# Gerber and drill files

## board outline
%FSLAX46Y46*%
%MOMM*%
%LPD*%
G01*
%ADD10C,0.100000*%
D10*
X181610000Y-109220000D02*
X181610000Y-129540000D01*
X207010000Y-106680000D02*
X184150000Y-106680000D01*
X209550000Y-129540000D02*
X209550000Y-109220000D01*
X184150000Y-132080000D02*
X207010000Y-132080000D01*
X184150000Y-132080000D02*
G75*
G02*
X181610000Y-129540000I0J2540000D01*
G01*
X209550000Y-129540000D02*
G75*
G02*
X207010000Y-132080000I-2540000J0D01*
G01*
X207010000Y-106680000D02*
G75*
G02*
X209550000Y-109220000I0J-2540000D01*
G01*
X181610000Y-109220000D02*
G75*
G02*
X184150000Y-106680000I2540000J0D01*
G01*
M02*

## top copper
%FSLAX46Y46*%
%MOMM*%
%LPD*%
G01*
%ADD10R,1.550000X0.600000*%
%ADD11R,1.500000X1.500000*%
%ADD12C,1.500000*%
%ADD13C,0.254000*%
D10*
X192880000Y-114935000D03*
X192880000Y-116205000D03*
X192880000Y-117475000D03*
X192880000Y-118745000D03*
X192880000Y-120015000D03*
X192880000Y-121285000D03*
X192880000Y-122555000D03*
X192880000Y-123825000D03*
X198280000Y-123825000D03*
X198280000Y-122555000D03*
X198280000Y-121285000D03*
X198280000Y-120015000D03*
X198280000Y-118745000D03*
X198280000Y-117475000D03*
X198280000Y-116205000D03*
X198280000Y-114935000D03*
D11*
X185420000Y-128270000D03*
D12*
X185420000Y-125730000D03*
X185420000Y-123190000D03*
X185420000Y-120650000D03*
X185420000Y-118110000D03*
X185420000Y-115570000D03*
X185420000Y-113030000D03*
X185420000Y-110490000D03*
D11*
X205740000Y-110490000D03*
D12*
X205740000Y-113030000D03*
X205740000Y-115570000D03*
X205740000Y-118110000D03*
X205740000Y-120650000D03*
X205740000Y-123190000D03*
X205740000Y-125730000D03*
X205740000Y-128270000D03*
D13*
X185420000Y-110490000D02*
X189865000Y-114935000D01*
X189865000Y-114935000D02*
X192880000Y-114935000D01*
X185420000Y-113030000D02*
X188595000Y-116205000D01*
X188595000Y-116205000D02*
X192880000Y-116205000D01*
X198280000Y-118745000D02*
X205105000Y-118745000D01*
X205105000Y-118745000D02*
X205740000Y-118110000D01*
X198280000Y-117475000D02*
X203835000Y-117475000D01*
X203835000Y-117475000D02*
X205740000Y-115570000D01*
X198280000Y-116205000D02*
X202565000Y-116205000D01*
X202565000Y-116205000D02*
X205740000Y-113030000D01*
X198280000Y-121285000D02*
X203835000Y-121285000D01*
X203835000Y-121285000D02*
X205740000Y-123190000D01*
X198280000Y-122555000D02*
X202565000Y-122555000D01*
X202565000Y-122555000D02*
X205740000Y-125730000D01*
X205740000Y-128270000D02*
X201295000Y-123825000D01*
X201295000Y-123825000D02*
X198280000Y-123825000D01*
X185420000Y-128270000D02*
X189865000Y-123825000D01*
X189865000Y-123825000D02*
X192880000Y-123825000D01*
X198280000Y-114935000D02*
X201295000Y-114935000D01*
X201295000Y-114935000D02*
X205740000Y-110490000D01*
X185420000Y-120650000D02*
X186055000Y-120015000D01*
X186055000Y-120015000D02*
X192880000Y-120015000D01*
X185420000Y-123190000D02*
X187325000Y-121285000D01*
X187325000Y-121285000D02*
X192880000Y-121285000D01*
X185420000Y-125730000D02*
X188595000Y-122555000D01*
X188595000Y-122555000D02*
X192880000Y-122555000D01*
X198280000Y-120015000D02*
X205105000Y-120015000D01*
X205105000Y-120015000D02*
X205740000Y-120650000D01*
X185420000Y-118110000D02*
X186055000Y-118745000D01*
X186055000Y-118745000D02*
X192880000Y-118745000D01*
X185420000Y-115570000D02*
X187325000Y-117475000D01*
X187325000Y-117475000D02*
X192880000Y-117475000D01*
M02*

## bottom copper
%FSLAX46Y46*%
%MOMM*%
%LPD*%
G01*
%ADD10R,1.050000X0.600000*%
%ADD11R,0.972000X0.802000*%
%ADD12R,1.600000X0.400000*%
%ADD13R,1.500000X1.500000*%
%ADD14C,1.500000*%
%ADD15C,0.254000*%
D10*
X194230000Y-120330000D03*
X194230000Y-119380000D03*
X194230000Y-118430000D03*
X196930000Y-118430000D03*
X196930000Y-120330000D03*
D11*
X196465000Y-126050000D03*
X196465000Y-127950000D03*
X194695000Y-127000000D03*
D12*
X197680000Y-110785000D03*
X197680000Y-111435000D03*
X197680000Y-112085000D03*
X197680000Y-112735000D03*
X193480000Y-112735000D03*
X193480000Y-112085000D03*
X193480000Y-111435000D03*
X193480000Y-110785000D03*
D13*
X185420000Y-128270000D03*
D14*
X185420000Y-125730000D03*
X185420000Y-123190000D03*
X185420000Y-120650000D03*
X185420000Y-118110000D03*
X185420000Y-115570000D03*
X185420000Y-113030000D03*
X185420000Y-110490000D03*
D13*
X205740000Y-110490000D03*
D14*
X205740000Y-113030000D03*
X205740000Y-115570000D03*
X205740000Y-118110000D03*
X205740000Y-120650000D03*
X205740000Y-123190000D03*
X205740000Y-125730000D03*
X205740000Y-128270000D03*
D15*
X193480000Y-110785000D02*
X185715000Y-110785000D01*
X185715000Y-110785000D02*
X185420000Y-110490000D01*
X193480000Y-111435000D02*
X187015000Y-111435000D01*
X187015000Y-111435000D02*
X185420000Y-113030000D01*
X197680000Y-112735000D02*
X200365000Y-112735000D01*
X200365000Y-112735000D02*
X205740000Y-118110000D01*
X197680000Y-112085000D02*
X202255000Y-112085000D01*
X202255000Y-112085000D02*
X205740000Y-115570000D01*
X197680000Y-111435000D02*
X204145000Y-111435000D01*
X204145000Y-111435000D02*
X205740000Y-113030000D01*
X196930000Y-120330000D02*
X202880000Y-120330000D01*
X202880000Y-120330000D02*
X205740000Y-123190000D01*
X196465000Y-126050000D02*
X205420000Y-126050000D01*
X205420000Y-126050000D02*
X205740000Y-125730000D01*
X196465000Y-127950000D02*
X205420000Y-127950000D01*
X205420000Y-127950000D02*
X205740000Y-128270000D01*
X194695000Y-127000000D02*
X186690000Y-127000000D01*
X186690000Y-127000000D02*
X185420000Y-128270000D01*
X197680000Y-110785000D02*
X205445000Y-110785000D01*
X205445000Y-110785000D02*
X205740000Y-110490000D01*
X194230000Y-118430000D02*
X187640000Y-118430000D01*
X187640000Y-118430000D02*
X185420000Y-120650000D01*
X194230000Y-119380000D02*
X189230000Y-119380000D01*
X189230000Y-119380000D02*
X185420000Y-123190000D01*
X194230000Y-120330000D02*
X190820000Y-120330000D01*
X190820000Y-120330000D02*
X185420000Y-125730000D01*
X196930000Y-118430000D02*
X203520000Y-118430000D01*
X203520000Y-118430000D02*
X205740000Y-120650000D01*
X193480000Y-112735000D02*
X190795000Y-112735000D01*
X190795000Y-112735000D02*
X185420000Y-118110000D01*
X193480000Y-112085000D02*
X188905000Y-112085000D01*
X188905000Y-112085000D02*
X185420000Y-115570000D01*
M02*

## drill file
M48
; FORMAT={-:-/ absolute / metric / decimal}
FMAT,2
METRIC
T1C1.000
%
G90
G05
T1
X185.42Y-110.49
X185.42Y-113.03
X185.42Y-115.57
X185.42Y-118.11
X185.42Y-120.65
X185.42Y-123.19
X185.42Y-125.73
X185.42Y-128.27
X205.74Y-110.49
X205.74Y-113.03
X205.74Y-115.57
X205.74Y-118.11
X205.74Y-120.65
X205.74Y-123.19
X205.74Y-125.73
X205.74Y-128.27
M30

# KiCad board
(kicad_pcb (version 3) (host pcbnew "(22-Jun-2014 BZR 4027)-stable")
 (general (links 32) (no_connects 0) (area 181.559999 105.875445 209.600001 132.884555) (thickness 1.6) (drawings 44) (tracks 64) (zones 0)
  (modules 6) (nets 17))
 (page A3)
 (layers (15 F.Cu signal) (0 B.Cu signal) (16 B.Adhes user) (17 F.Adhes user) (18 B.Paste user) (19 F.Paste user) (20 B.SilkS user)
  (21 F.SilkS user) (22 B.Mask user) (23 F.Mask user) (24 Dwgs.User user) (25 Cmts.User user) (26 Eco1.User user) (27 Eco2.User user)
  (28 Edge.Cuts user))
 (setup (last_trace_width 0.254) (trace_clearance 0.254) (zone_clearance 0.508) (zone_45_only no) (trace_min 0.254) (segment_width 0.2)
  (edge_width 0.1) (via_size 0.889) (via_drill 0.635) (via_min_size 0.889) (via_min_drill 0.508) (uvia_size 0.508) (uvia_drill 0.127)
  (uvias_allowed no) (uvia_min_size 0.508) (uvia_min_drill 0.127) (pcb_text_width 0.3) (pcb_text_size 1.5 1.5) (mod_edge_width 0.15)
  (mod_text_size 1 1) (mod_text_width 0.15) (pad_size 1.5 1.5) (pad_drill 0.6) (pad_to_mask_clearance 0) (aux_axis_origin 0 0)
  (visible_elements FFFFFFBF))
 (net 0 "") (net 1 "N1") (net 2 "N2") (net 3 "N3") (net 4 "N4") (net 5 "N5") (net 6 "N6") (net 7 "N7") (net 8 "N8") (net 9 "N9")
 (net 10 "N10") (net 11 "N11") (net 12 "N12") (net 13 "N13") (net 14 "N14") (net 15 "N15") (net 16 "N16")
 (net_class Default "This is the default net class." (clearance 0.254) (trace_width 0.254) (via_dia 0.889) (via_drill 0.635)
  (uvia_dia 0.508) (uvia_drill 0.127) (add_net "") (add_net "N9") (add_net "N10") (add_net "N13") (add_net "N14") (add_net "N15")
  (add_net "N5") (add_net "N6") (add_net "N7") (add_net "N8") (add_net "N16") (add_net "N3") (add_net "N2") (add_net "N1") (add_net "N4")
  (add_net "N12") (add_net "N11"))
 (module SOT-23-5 (layer B.Cu) (at 195.58 119.38 90) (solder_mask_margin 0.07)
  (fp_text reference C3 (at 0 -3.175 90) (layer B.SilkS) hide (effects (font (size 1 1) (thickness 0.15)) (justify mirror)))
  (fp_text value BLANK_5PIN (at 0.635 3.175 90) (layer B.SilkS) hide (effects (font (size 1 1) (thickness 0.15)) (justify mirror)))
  (pad 1 smd rect (at -0.95 -1.35 90) (size 0.6 1.05) (layers B.Cu B.Paste B.Mask) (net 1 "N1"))
  (pad 2 smd rect (at 0 -1.35 90) (size 0.6 1.05) (layers B.Cu B.Paste B.Mask) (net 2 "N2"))
  (pad 3 smd rect (at 0.95 -1.35 90) (size 0.6 1.05) (layers B.Cu B.Paste B.Mask) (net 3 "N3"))
  (pad 4 smd rect (at 0.95 1.35 90) (size 0.6 1.05) (layers B.Cu B.Paste B.Mask) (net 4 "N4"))
  (pad 5 smd rect (at -0.95 1.35 90) (size 0.6 1.05) (layers B.Cu B.Paste B.Mask) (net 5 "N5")))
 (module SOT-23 (layer B.Cu) (at 195.58 127 270) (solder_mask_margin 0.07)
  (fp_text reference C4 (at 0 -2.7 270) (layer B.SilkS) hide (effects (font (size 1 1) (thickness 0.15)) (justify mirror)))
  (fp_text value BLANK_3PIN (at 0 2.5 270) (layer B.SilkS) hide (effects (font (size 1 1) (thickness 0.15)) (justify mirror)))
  (pad 1 smd rect (at -0.95 -0.885 270) (size 0.802 0.972) (layers B.Cu B.Paste B.Mask) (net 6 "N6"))
  (pad 2 smd rect (at 0.95 -0.885 270) (size 0.802 0.972) (layers B.Cu B.Paste B.Mask) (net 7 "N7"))
  (pad 3 smd rect (at 0 0.885 270) (size 0.802 0.972) (layers B.Cu B.Paste B.Mask) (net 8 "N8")))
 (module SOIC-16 (layer F.Cu) (at 195.58 119.38 270)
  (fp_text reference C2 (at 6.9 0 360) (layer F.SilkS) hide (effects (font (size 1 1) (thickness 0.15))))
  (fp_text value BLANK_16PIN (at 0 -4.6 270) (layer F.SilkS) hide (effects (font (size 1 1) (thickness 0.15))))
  (pad 1 smd rect (at -4.445 2.7 270) (size 0.6 1.55) (layers F.Cu F.Paste F.Mask) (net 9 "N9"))
  (pad 2 smd rect (at -3.175 2.7 270) (size 0.6 1.55) (layers F.Cu F.Paste F.Mask) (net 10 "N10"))
  (pad 3 smd rect (at -1.905 2.7 270) (size 0.6 1.55) (layers F.Cu F.Paste F.Mask) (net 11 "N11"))
  (pad 4 smd rect (at -0.635 2.7 270) (size 0.6 1.55) (layers F.Cu F.Paste F.Mask) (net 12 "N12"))
  (pad 5 smd rect (at 0.635 2.7 270) (size 0.6 1.55) (layers F.Cu F.Paste F.Mask) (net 3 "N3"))
  (pad 6 smd rect (at 1.905 2.7 270) (size 0.6 1.55) (layers F.Cu F.Paste F.Mask) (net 2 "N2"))
  (pad 7 smd rect (at 3.175 2.7 270) (size 0.6 1.55) (layers F.Cu F.Paste F.Mask) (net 1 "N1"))
  (pad 8 smd rect (at 4.445 2.7 270) (size 0.6 1.55) (layers F.Cu F.Paste F.Mask) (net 8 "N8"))
  (pad 9 smd rect (at 4.445 -2.7 270) (size 0.6 1.55) (layers F.Cu F.Paste F.Mask) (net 7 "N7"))
  (pad 10 smd rect (at 3.175 -2.7 270) (size 0.6 1.55) (layers F.Cu F.Paste F.Mask) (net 6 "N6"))
  (pad 11 smd rect (at 1.905 -2.7 270) (size 0.6 1.55) (layers F.Cu F.Paste F.Mask) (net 5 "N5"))
  (pad 12 smd rect (at 0.635 -2.7 270) (size 0.6 1.55) (layers F.Cu F.Paste F.Mask) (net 4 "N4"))
  (pad 13 smd rect (at -0.635 -2.7 270) (size 0.6 1.55) (layers F.Cu F.Paste F.Mask) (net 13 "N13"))
  (pad 14 smd rect (at -1.905 -2.7 270) (size 0.6 1.55) (layers F.Cu F.Paste F.Mask) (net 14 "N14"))
  (pad 15 smd rect (at -3.175 -2.7 270) (size 0.6 1.55) (layers F.Cu F.Paste F.Mask) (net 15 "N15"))
  (pad 16 smd rect (at -4.445 -2.7 270) (size 0.6 1.55) (layers F.Cu F.Paste F.Mask) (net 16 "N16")))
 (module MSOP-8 (layer B.Cu) (at 195.58 111.76 270) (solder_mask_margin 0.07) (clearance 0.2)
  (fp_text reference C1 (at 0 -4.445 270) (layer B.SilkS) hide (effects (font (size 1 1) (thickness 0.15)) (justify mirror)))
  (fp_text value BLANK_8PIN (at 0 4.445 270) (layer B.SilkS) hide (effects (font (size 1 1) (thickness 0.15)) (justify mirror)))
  (pad 1 smd rect (at -0.975 -2.1 270) (size 0.4 1.6) (layers B.Cu B.Paste B.Mask) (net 16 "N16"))
  (pad 2 smd rect (at -0.325 -2.1 270) (size 0.4 1.6) (layers B.Cu B.Paste B.Mask) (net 15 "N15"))
  (pad 3 smd rect (at 0.325 -2.1 270) (size 0.4 1.6) (layers B.Cu B.Paste B.Mask) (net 14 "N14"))
  (pad 4 smd rect (at 0.975 -2.1 270) (size 0.4 1.6) (layers B.Cu B.Paste B.Mask) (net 13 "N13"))
  (pad 5 smd rect (at 0.975 2.1 270) (size 0.4 1.6) (layers B.Cu B.Paste B.Mask) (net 12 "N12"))
  (pad 6 smd rect (at 0.325 2.1 270) (size 0.4 1.6) (layers B.Cu B.Paste B.Mask) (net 11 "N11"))
  (pad 7 smd rect (at -0.325 2.1 270) (size 0.4 1.6) (layers B.Cu B.Paste B.Mask) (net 10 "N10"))
  (pad 8 smd rect (at -0.975 2.1 270) (size 0.4 1.6) (layers B.Cu B.Paste B.Mask) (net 9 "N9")))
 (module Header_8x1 (layer F.Cu) (at 185.42 119.38 90)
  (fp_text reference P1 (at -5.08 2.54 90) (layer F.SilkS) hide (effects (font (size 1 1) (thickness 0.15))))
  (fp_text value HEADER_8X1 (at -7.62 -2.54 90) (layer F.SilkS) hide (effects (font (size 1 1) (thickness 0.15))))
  (pad 1 thru_hole rect (at -8.89 0 90) (size 1.5 1.5) (drill 1) (layers *.Cu *.Mask F.SilkS) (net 8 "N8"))
  (pad 2 thru_hole circle (at -6.35 0 90) (size 1.5 1.5) (drill 1) (layers *.Cu *.Mask F.SilkS) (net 1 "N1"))
  (pad 3 thru_hole circle (at -3.81 0 90) (size 1.5 1.5) (drill 1) (layers *.Cu *.Mask F.SilkS) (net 2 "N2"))
  (pad 4 thru_hole circle (at -1.27 0 90) (size 1.5 1.5) (drill 1) (layers *.Cu *.Mask F.SilkS) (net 3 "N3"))
  (pad 5 thru_hole circle (at 1.27 0 90) (size 1.5 1.5) (drill 1) (layers *.Cu *.Mask F.SilkS) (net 12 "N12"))
  (pad 6 thru_hole circle (at 3.81 0 90) (size 1.5 1.5) (drill 1) (layers *.Cu *.Mask F.SilkS) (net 11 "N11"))
  (pad 7 thru_hole circle (at 6.35 0 90) (size 1.5 1.5) (drill 1) (layers *.Cu *.Mask F.SilkS) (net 10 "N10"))
  (pad 8 thru_hole circle (at 8.89 0 90) (size 1.5 1.5) (drill 1) (layers *.Cu *.Mask F.SilkS) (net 9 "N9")))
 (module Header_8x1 (layer F.Cu) (at 205.74 119.38 270)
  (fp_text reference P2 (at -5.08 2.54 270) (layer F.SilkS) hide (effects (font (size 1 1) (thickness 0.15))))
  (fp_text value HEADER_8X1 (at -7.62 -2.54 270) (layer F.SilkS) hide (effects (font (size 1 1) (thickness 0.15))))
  (pad 1 thru_hole rect (at -8.89 0 270) (size 1.5 1.5) (drill 1) (layers *.Cu *.Mask F.SilkS) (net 16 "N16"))
  (pad 2 thru_hole circle (at -6.35 0 270) (size 1.5 1.5) (drill 1) (layers *.Cu *.Mask F.SilkS) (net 15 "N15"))
  (pad 3 thru_hole circle (at -3.81 0 270) (size 1.5 1.5) (drill 1) (layers *.Cu *.Mask F.SilkS) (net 14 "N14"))
  (pad 4 thru_hole circle (at -1.27 0 270) (size 1.5 1.5) (drill 1) (layers *.Cu *.Mask F.SilkS) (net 13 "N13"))
  (pad 5 thru_hole circle (at 1.27 0 270) (size 1.5 1.5) (drill 1) (layers *.Cu *.Mask F.SilkS) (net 4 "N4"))
  (pad 6 thru_hole circle (at 3.81 0 270) (size 1.5 1.5) (drill 1) (layers *.Cu *.Mask F.SilkS) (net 5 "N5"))
  (pad 7 thru_hole circle (at 6.35 0 270) (size 1.5 1.5) (drill 1) (layers *.Cu *.Mask F.SilkS) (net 6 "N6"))
  (pad 8 thru_hole circle (at 8.89 0 270) (size 1.5 1.5) (drill 1) (layers *.Cu *.Mask F.SilkS) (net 7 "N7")))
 (gr_line (start 181.61 109.22) (end 181.61 129.54) (angle 90) (layer Edge.Cuts) (width 0.1))
 (gr_line (start 207.01 106.68) (end 184.15 106.68) (angle 90) (layer Edge.Cuts) (width 0.1))
 (gr_line (start 209.55 129.54) (end 209.55 109.22) (angle 90) (layer Edge.Cuts) (width 0.1))
 (gr_line (start 184.15 132.08) (end 207.01 132.08) (angle 90) (layer Edge.Cuts) (width 0.1))
 (gr_arc (start 184.15 129.54) (end 184.15 132.08) (angle 90) (layer Edge.Cuts) (width 0.1))
 (gr_arc (start 207.01 129.54) (end 209.55 129.54) (angle 90) (layer Edge.Cuts) (width 0.1))
 (gr_arc (start 207.01 109.22) (end 207.01 106.68) (angle 90) (layer Edge.Cuts) (width 0.1))
 (gr_arc (start 184.15 109.22) (end 181.61 109.22) (angle 90) (layer Edge.Cuts) (width 0.1))
 (segment (start 185.42 110.49) (end 189.865 114.935) (width 0.254) (layer F.Cu) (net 9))
 (segment (start 189.865 114.935) (end 192.88 114.935) (width 0.254) (layer F.Cu) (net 9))
 (segment (start 193.48 110.785) (end 185.715 110.785) (width 0.254) (layer B.Cu) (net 9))
 (segment (start 185.715 110.785) (end 185.42 110.49) (width 0.254) (layer B.Cu) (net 9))
 (segment (start 185.42 113.03) (end 188.595 116.205) (width 0.254) (layer F.Cu) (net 10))
 (segment (start 188.595 116.205) (end 192.88 116.205) (width 0.254) (layer F.Cu) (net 10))
 (segment (start 193.48 111.435) (end 187.015 111.435) (width 0.254) (layer B.Cu) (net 10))
 (segment (start 187.015 111.435) (end 185.42 113.03) (width 0.254) (layer B.Cu) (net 10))
 (segment (start 198.28 118.745) (end 205.105 118.745) (width 0.254) (layer F.Cu) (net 13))
 (segment (start 205.105 118.745) (end 205.74 118.11) (width 0.254) (layer F.Cu) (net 13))
 (segment (start 197.68 112.735) (end 200.365 112.735) (width 0.254) (layer B.Cu) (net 13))
 (segment (start 200.365 112.735) (end 205.74 118.11) (width 0.254) (layer B.Cu) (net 13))
 (segment (start 198.28 117.475) (end 203.835 117.475) (width 0.254) (layer F.Cu) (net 14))
 (segment (start 203.835 117.475) (end 205.74 115.57) (width 0.254) (layer F.Cu) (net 14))
 (segment (start 197.68 112.085) (end 202.255 112.085) (width 0.254) (layer B.Cu) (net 14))
 (segment (start 202.255 112.085) (end 205.74 115.57) (width 0.254) (layer B.Cu) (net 14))
 (segment (start 198.28 116.205) (end 202.565 116.205) (width 0.254) (layer F.Cu) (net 15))
 (segment (start 202.565 116.205) (end 205.74 113.03) (width 0.254) (layer F.Cu) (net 15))
 (segment (start 197.68 111.435) (end 204.145 111.435) (width 0.254) (layer B.Cu) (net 15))
 (segment (start 204.145 111.435) (end 205.74 113.03) (width 0.254) (layer B.Cu) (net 15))
 (segment (start 198.28 121.285) (end 203.835 121.285) (width 0.254) (layer F.Cu) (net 5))
 (segment (start 203.835 121.285) (end 205.74 123.19) (width 0.254) (layer F.Cu) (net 5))
 (segment (start 196.93 120.33) (end 202.88 120.33) (width 0.254) (layer B.Cu) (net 5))
 (segment (start 202.88 120.33) (end 205.74 123.19) (width 0.254) (layer B.Cu) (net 5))
 (segment (start 198.28 122.555) (end 202.565 122.555) (width 0.254) (layer F.Cu) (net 6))
 (segment (start 202.565 122.555) (end 205.74 125.73) (width 0.254) (layer F.Cu) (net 6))
 (segment (start 196.465 126.05) (end 205.42 126.05) (width 0.254) (layer B.Cu) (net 6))
 (segment (start 205.42 126.05) (end 205.74 125.73) (width 0.254) (layer B.Cu) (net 6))
 (segment (start 205.74 128.27) (end 201.295 123.825) (width 0.254) (layer F.Cu) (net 7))
 (segment (start 201.295 123.825) (end 198.28 123.825) (width 0.254) (layer F.Cu) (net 7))
 (segment (start 196.465 127.95) (end 205.42 127.95) (width 0.254) (layer B.Cu) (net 7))
 (segment (start 205.42 127.95) (end 205.74 128.27) (width 0.254) (layer B.Cu) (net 7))
 (segment (start 185.42 128.27) (end 189.865 123.825) (width 0.254) (layer F.Cu) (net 8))
 (segment (start 189.865 123.825) (end 192.88 123.825) (width 0.254) (layer F.Cu) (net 8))
 (segment (start 194.695 127) (end 186.69 127) (width 0.254) (layer B.Cu) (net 8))
 (segment (start 186.69 127) (end 185.42 128.27) (width 0.254) (layer B.Cu) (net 8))
 (segment (start 198.28 114.935) (end 201.295 114.935) (width 0.254) (layer F.Cu) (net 16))
 (segment (start 201.295 114.935) (end 205.74 110.49) (width 0.254) (layer F.Cu) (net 16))
 (segment (start 197.68 110.785) (end 205.445 110.785) (width 0.254) (layer B.Cu) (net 16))
 (segment (start 205.445 110.785) (end 205.74 110.49) (width 0.254) (layer B.Cu) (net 16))
 (segment (start 185.42 120.65) (end 186.055 120.015) (width 0.254) (layer F.Cu) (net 3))
 (segment (start 186.055 120.015) (end 192.88 120.015) (width 0.254) (layer F.Cu) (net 3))
 (segment (start 194.23 118.43) (end 187.64 118.43) (width 0.254) (layer B.Cu) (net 3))
 (segment (start 187.64 118.43) (end 185.42 120.65) (width 0.254) (layer B.Cu) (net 3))
 (segment (start 185.42 123.19) (end 187.325 121.285) (width 0.254) (layer F.Cu) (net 2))
 (segment (start 187.325 121.285) (end 192.88 121.285) (width 0.254) (layer F.Cu) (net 2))
 (segment (start 194.23 119.38) (end 189.23 119.38) (width 0.254) (layer B.Cu) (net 2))
 (segment (start 189.23 119.38) (end 185.42 123.19) (width 0.254) (layer B.Cu) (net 2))
 (segment (start 185.42 125.73) (end 188.595 122.555) (width 0.254) (layer F.Cu) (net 1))
 (segment (start 188.595 122.555) (end 192.88 122.555) (width 0.254) (layer F.Cu) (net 1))
 (segment (start 194.23 120.33) (end 190.82 120.33) (width 0.254) (layer B.Cu) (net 1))
 (segment (start 190.82 120.33) (end 185.42 125.73) (width 0.254) (layer B.Cu) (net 1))
 (segment (start 198.28 120.015) (end 205.105 120.015) (width 0.254) (layer F.Cu) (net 4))
 (segment (start 205.105 120.015) (end 205.74 120.65) (width 0.254) (layer F.Cu) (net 4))
 (segment (start 196.93 118.43) (end 203.52 118.43) (width 0.254) (layer B.Cu) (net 4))
 (segment (start 203.52 118.43) (end 205.74 120.65) (width 0.254) (layer B.Cu) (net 4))
 (segment (start 185.42 118.11) (end 186.055 118.745) (width 0.254) (layer F.Cu) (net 12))
 (segment (start 186.055 118.745) (end 192.88 118.745) (width 0.254) (layer F.Cu) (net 12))
 (segment (start 193.48 112.735) (end 190.795 112.735) (width 0.254) (layer B.Cu) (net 12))
 (segment (start 190.795 112.735) (end 185.42 118.11) (width 0.254) (layer B.Cu) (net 12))
 (segment (start 185.42 115.57) (end 187.325 117.475) (width 0.254) (layer F.Cu) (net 11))
 (segment (start 187.325 117.475) (end 192.88 117.475) (width 0.254) (layer F.Cu) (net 11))
 (segment (start 193.48 112.085) (end 188.905 112.085) (width 0.254) (layer B.Cu) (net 11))
 (segment (start 188.905 112.085) (end 185.42 115.57) (width 0.254) (layer B.Cu) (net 11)))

